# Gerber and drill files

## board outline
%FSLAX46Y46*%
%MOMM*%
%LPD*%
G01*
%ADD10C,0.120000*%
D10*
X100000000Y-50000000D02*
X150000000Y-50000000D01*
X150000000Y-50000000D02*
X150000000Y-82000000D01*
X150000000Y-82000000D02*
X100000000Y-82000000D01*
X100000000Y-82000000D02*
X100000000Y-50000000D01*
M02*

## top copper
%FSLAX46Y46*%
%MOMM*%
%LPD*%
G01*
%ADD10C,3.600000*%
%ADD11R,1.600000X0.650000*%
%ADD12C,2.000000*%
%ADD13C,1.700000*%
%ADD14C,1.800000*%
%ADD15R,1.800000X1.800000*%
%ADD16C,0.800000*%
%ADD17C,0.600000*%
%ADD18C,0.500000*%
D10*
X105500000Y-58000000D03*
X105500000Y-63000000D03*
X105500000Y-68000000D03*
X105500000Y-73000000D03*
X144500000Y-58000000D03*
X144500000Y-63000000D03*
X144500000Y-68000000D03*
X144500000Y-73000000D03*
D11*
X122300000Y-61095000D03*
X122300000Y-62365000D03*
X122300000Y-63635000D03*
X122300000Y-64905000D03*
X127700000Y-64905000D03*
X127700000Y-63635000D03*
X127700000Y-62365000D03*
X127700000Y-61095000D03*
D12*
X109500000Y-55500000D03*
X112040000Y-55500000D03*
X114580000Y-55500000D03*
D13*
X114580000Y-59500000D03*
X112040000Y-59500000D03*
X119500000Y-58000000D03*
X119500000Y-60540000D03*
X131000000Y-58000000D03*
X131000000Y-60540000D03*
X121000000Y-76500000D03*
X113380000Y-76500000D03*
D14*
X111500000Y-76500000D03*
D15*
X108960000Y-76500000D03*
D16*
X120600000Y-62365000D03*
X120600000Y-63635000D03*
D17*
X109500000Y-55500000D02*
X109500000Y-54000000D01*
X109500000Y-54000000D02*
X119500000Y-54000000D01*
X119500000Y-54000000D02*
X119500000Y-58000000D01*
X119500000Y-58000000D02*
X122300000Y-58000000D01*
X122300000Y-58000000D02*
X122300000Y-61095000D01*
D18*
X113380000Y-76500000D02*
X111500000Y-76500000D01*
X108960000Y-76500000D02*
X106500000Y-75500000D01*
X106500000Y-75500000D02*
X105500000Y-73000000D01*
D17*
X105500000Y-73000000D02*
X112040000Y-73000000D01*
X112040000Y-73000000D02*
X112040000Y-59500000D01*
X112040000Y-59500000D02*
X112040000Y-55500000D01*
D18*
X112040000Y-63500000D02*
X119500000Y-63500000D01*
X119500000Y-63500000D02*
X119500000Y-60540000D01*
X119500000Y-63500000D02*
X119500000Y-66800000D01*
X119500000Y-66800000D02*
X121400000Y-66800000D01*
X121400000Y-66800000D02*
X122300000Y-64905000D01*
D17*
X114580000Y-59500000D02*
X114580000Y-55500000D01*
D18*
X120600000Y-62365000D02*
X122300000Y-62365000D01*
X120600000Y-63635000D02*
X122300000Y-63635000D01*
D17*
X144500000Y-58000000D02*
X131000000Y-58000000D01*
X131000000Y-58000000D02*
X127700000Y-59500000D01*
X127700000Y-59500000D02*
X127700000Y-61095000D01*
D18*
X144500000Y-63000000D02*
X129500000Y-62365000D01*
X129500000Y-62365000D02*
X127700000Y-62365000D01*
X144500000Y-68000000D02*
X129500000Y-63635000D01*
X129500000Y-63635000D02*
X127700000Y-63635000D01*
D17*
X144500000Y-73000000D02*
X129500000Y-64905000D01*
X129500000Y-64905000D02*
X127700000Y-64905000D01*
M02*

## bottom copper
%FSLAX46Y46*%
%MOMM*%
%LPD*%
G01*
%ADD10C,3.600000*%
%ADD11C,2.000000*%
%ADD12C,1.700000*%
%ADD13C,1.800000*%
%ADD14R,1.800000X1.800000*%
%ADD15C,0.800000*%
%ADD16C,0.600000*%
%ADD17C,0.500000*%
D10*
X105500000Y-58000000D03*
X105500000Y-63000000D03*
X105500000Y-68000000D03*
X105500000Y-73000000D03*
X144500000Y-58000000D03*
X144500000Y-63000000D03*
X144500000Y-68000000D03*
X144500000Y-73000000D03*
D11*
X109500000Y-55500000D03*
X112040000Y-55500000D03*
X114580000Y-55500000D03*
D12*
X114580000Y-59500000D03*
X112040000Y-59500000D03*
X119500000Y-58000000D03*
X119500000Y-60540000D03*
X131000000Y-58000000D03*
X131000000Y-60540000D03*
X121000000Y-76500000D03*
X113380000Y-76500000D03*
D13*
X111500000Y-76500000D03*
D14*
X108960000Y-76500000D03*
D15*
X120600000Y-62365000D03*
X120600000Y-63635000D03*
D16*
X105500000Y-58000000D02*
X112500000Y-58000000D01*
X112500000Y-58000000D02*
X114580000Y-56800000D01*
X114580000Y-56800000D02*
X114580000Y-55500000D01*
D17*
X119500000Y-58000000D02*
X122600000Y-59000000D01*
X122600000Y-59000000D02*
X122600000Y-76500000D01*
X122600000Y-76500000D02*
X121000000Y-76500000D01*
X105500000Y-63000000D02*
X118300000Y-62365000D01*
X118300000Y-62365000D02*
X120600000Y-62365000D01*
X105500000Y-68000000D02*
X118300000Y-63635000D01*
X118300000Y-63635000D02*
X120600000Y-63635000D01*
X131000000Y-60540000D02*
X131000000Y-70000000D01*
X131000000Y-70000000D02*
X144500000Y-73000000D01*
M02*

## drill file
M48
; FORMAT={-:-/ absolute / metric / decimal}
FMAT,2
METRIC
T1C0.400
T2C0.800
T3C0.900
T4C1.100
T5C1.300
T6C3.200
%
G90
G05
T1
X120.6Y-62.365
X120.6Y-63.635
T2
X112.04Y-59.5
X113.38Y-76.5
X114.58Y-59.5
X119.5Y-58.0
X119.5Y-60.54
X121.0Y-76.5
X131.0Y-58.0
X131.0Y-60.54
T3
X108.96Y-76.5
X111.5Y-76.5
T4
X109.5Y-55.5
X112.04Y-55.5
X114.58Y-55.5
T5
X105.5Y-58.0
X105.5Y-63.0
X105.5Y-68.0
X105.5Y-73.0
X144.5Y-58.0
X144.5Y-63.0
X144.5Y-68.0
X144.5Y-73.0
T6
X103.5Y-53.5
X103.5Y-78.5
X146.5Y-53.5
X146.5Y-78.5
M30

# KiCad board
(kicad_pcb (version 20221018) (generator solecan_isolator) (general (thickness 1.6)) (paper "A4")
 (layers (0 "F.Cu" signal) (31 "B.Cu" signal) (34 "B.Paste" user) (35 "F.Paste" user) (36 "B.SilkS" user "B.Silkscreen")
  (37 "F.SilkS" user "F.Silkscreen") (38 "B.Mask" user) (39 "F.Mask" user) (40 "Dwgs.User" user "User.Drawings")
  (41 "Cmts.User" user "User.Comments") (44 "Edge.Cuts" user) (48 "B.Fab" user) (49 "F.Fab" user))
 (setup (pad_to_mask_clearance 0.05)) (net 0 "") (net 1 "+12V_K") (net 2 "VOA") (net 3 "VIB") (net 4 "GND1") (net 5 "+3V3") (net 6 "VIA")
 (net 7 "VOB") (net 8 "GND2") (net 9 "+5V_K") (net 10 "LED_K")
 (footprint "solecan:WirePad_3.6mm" (layer "F.Cu") (at 105.500 58.000)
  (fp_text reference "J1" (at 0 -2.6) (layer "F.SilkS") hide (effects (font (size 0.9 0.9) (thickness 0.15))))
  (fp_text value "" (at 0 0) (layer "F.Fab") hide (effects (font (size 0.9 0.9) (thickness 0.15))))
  (pad "1" thru_hole circle (at 0.000 0.000) (size 3.6 3.6) (drill 1.3) (layers "*.Cu" "*.Mask") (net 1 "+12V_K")))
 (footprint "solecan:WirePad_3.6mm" (layer "F.Cu") (at 105.500 63.000)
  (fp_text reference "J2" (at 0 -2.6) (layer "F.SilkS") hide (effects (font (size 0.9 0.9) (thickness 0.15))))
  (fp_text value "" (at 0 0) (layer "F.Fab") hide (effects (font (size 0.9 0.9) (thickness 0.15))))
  (pad "1" thru_hole circle (at 0.000 0.000) (size 3.6 3.6) (drill 1.3) (layers "*.Cu" "*.Mask") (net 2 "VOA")))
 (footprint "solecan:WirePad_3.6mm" (layer "F.Cu") (at 105.500 68.000)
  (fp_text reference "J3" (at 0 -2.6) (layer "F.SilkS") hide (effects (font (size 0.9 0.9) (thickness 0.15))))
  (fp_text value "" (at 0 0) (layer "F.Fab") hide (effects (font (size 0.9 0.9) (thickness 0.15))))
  (pad "1" thru_hole circle (at 0.000 0.000) (size 3.6 3.6) (drill 1.3) (layers "*.Cu" "*.Mask") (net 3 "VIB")))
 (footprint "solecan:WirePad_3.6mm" (layer "F.Cu") (at 105.500 73.000)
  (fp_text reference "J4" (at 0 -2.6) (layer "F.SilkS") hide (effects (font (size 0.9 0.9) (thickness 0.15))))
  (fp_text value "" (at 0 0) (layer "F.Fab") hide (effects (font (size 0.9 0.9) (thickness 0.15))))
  (pad "1" thru_hole circle (at 0.000 0.000) (size 3.6 3.6) (drill 1.3) (layers "*.Cu" "*.Mask") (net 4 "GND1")))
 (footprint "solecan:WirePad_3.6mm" (layer "F.Cu") (at 144.500 58.000)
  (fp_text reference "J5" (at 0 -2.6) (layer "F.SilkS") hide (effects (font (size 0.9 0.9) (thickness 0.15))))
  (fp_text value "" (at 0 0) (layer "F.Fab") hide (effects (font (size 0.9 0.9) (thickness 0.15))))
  (pad "1" thru_hole circle (at 0.000 0.000) (size 3.6 3.6) (drill 1.3) (layers "*.Cu" "*.Mask") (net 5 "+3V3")))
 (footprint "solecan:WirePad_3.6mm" (layer "F.Cu") (at 144.500 63.000)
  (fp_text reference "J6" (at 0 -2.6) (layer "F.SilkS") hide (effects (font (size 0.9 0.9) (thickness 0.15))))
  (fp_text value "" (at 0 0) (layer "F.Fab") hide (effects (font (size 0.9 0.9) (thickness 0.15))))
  (pad "1" thru_hole circle (at 0.000 0.000) (size 3.6 3.6) (drill 1.3) (layers "*.Cu" "*.Mask") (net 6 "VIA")))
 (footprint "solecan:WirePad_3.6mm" (layer "F.Cu") (at 144.500 68.000)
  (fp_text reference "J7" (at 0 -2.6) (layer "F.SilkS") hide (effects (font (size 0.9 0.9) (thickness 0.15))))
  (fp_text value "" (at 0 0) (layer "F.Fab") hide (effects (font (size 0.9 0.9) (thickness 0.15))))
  (pad "1" thru_hole circle (at 0.000 0.000) (size 3.6 3.6) (drill 1.3) (layers "*.Cu" "*.Mask") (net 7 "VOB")))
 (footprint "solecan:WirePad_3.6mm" (layer "F.Cu") (at 144.500 73.000)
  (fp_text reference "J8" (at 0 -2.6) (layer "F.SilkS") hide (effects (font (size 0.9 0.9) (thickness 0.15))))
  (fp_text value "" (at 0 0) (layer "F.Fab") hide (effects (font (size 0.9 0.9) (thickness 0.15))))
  (pad "1" thru_hole circle (at 0.000 0.000) (size 3.6 3.6) (drill 1.3) (layers "*.Cu" "*.Mask") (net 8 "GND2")))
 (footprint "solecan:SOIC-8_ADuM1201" (layer "F.Cu") (at 125.000 63.000)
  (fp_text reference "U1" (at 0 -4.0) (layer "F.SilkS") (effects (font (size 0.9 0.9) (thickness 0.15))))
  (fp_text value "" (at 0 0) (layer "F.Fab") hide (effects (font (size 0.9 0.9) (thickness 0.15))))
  (pad "1" smd rect (at -2.700 -1.905) (size 1.6 0.65) (layers "F.Cu" "F.Paste" "F.Mask") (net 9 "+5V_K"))
  (pad "2" smd rect (at -2.700 -0.635) (size 1.6 0.65) (layers "F.Cu" "F.Paste" "F.Mask") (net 2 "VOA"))
  (pad "3" smd rect (at -2.700 0.635) (size 1.6 0.65) (layers "F.Cu" "F.Paste" "F.Mask") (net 3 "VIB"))
  (pad "4" smd rect (at -2.700 1.905) (size 1.6 0.65) (layers "F.Cu" "F.Paste" "F.Mask") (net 4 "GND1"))
  (pad "5" smd rect (at 2.700 1.905) (size 1.6 0.65) (layers "F.Cu" "F.Paste" "F.Mask") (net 8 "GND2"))
  (pad "6" smd rect (at 2.700 0.635) (size 1.6 0.65) (layers "F.Cu" "F.Paste" "F.Mask") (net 7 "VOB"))
  (pad "7" smd rect (at 2.700 -0.635) (size 1.6 0.65) (layers "F.Cu" "F.Paste" "F.Mask") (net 6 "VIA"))
  (pad "8" smd rect (at 2.700 -1.905) (size 1.6 0.65) (layers "F.Cu" "F.Paste" "F.Mask") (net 5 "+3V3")))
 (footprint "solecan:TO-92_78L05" (layer "F.Cu") (at 112.040 55.500)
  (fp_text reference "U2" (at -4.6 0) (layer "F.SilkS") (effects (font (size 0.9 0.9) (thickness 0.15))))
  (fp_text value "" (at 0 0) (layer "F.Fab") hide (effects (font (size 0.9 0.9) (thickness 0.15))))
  (pad "1" thru_hole circle (at -2.540 0.000) (size 2.0 2.0) (drill 1.1) (layers "*.Cu" "*.Mask") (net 9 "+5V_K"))
  (pad "2" thru_hole circle (at 0.000 0.000) (size 2.0 2.0) (drill 1.1) (layers "*.Cu" "*.Mask") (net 4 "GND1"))
  (pad "3" thru_hole circle (at 2.540 0.000) (size 2.0 2.0) (drill 1.1) (layers "*.Cu" "*.Mask") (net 1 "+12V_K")))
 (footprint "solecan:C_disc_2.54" (layer "F.Cu") (at 113.310 59.500)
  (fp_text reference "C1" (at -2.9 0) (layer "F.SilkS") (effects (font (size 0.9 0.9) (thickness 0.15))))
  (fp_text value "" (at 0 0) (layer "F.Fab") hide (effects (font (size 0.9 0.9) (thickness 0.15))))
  (pad "1" thru_hole circle (at 1.270 0.000) (size 1.7 1.7) (drill 0.8) (layers "*.Cu" "*.Mask") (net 1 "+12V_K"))
  (pad "2" thru_hole circle (at -1.270 0.000) (size 1.7 1.7) (drill 0.8) (layers "*.Cu" "*.Mask") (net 4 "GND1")))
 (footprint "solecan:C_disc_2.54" (layer "F.Cu") (at 119.500 59.270)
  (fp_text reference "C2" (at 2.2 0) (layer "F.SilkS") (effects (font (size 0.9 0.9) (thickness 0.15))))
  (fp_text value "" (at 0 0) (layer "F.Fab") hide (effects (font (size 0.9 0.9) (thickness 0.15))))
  (pad "1" thru_hole circle (at 0.000 -1.270) (size 1.7 1.7) (drill 0.8) (layers "*.Cu" "*.Mask") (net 9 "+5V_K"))
  (pad "2" thru_hole circle (at 0.000 1.270) (size 1.7 1.7) (drill 0.8) (layers "*.Cu" "*.Mask") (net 4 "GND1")))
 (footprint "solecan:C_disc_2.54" (layer "F.Cu") (at 131.000 59.270)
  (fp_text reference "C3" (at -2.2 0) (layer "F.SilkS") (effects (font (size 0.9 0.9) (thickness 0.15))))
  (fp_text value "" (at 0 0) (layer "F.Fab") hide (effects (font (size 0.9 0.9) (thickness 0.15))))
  (pad "1" thru_hole circle (at 0.000 -1.270) (size 1.7 1.7) (drill 0.8) (layers "*.Cu" "*.Mask") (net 5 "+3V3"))
  (pad "2" thru_hole circle (at 0.000 1.270) (size 1.7 1.7) (drill 0.8) (layers "*.Cu" "*.Mask") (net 8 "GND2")))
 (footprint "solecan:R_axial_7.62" (layer "F.Cu") (at 117.190 76.500)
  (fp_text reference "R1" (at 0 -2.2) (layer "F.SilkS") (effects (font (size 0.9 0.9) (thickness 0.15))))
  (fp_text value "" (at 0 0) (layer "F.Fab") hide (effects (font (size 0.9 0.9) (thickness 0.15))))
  (pad "1" thru_hole circle (at 3.810 0.000) (size 1.7 1.7) (drill 0.8) (layers "*.Cu" "*.Mask") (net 9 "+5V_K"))
  (pad "2" thru_hole circle (at -3.810 0.000) (size 1.7 1.7) (drill 0.8) (layers "*.Cu" "*.Mask") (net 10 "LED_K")))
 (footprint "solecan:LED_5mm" (layer "F.Cu") (at 110.230 76.500)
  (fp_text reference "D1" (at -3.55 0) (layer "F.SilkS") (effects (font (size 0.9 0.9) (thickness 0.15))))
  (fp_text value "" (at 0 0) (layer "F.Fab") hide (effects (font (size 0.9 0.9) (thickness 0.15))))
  (pad "1" thru_hole circle (at 1.270 0.000) (size 1.8 1.8) (drill 0.9) (layers "*.Cu" "*.Mask") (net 10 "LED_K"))
  (pad "2" thru_hole rect (at -1.270 0.000) (size 1.8 1.8) (drill 0.9) (layers "*.Cu" "*.Mask") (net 4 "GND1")))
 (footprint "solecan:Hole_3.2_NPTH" (layer "F.Cu") (at 103.500 53.500)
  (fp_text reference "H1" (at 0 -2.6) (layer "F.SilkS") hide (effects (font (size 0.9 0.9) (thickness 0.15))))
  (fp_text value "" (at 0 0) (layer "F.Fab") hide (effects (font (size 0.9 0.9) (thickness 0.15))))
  (pad "" np_thru_hole circle (at 0 0) (size 3.2 3.2) (drill 3.2) (layers "*.Cu" "*.Mask")))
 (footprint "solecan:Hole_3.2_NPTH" (layer "F.Cu") (at 103.500 78.500)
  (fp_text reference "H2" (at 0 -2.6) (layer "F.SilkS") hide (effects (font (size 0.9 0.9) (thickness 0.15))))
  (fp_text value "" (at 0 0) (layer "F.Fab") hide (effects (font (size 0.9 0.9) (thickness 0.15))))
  (pad "" np_thru_hole circle (at 0 0) (size 3.2 3.2) (drill 3.2) (layers "*.Cu" "*.Mask")))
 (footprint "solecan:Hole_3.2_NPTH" (layer "F.Cu") (at 146.500 53.500)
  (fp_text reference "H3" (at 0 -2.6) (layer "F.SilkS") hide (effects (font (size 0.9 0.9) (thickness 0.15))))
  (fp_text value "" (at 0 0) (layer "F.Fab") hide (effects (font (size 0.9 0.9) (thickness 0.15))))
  (pad "" np_thru_hole circle (at 0 0) (size 3.2 3.2) (drill 3.2) (layers "*.Cu" "*.Mask")))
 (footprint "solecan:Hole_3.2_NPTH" (layer "F.Cu") (at 146.500 78.500)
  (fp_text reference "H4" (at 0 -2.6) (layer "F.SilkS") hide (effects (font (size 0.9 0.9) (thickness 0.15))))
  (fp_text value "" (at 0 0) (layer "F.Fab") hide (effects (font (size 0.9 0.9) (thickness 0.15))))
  (pad "" np_thru_hole circle (at 0 0) (size 3.2 3.2) (drill 3.2) (layers "*.Cu" "*.Mask")))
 (segment (start 105.500 58.000) (end 112.500 58.000) (width 0.6) (layer "B.Cu") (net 1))
 (segment (start 112.500 58.000) (end 114.580 56.800) (width 0.6) (layer "B.Cu") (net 1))
 (segment (start 114.580 56.800) (end 114.580 55.500) (width 0.6) (layer "B.Cu") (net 1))
 (segment (start 109.500 55.500) (end 109.500 54.000) (width 0.6) (layer "F.Cu") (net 9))
 (segment (start 109.500 54.000) (end 119.500 54.000) (width 0.6) (layer "F.Cu") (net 9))
 (segment (start 119.500 54.000) (end 119.500 58.000) (width 0.6) (layer "F.Cu") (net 9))
 (segment (start 119.500 58.000) (end 122.300 58.000) (width 0.6) (layer "F.Cu") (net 9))
 (segment (start 122.300 58.000) (end 122.300 61.095) (width 0.6) (layer "F.Cu") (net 9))
 (segment (start 119.500 58.000) (end 122.600 59.000) (width 0.5) (layer "B.Cu") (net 9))
 (segment (start 122.600 59.000) (end 122.600 76.500) (width 0.5) (layer "B.Cu") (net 9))
 (segment (start 122.600 76.500) (end 121.000 76.500) (width 0.5) (layer "B.Cu") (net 9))
 (segment (start 113.380 76.500) (end 111.500 76.500) (width 0.5) (layer "F.Cu") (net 10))
 (segment (start 108.960 76.500) (end 106.500 75.500) (width 0.5) (layer "F.Cu") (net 4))
 (segment (start 106.500 75.500) (end 105.500 73.000) (width 0.5) (layer "F.Cu") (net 4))
 (segment (start 105.500 73.000) (end 112.040 73.000) (width 0.6) (layer "F.Cu") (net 4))
 (segment (start 112.040 73.000) (end 112.040 59.500) (width 0.6) (layer "F.Cu") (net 4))
 (segment (start 112.040 59.500) (end 112.040 55.500) (width 0.6) (layer "F.Cu") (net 4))
 (segment (start 112.040 63.500) (end 119.500 63.500) (width 0.5) (layer "F.Cu") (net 4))
 (segment (start 119.500 63.500) (end 119.500 60.540) (width 0.5) (layer "F.Cu") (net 4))
 (segment (start 119.500 63.500) (end 119.500 66.800) (width 0.5) (layer "F.Cu") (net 4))
 (segment (start 119.500 66.800) (end 121.400 66.800) (width 0.5) (layer "F.Cu") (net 4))
 (segment (start 121.400 66.800) (end 122.300 64.905) (width 0.5) (layer "F.Cu") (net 4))
 (segment (start 114.580 59.500) (end 114.580 55.500) (width 0.6) (layer "F.Cu") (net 1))
 (segment (start 105.500 63.000) (end 118.300 62.365) (width 0.5) (layer "B.Cu") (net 2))
 (segment (start 118.300 62.365) (end 120.600 62.365) (width 0.5) (layer "B.Cu") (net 2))
 (via (at 120.600 62.365) (size 0.8) (drill 0.4) (layers "F.Cu" "B.Cu") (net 2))
 (segment (start 120.600 62.365) (end 122.300 62.365) (width 0.5) (layer "F.Cu") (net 2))
 (segment (start 105.500 68.000) (end 118.300 63.635) (width 0.5) (layer "B.Cu") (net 3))
 (segment (start 118.300 63.635) (end 120.600 63.635) (width 0.5) (layer "B.Cu") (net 3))
 (via (at 120.600 63.635) (size 0.8) (drill 0.4) (layers "F.Cu" "B.Cu") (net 3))
 (segment (start 120.600 63.635) (end 122.300 63.635) (width 0.5) (layer "F.Cu") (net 3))
 (segment (start 144.500 58.000) (end 131.000 58.000) (width 0.6) (layer "F.Cu") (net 5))
 (segment (start 131.000 58.000) (end 127.700 59.500) (width 0.6) (layer "F.Cu") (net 5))
 (segment (start 127.700 59.500) (end 127.700 61.095) (width 0.6) (layer "F.Cu") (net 5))
 (segment (start 144.500 63.000) (end 129.500 62.365) (width 0.5) (layer "F.Cu") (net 6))
 (segment (start 129.500 62.365) (end 127.700 62.365) (width 0.5) (layer "F.Cu") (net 6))
 (segment (start 144.500 68.000) (end 129.500 63.635) (width 0.5) (layer "F.Cu") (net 7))
 (segment (start 129.500 63.635) (end 127.700 63.635) (width 0.5) (layer "F.Cu") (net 7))
 (segment (start 144.500 73.000) (end 129.500 64.905) (width 0.6) (layer "F.Cu") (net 8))
 (segment (start 129.500 64.905) (end 127.700 64.905) (width 0.6) (layer "F.Cu") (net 8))
 (segment (start 131.000 60.540) (end 131.000 70.000) (width 0.5) (layer "B.Cu") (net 8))
 (segment (start 131.000 70.000) (end 144.500 73.000) (width 0.5) (layer "B.Cu") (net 8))
 (gr_line (start 100.000 50.000) (end 150.000 50.000) (stroke (width 0.12) (type solid)) (layer "Edge.Cuts"))
 (gr_line (start 150.000 50.000) (end 150.000 82.000) (stroke (width 0.12) (type solid)) (layer "Edge.Cuts"))
 (gr_line (start 150.000 82.000) (end 100.000 82.000) (stroke (width 0.12) (type solid)) (layer "Edge.Cuts"))
 (gr_line (start 100.000 82.000) (end 100.000 50.000) (stroke (width 0.12) (type solid)) (layer "Edge.Cuts")))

